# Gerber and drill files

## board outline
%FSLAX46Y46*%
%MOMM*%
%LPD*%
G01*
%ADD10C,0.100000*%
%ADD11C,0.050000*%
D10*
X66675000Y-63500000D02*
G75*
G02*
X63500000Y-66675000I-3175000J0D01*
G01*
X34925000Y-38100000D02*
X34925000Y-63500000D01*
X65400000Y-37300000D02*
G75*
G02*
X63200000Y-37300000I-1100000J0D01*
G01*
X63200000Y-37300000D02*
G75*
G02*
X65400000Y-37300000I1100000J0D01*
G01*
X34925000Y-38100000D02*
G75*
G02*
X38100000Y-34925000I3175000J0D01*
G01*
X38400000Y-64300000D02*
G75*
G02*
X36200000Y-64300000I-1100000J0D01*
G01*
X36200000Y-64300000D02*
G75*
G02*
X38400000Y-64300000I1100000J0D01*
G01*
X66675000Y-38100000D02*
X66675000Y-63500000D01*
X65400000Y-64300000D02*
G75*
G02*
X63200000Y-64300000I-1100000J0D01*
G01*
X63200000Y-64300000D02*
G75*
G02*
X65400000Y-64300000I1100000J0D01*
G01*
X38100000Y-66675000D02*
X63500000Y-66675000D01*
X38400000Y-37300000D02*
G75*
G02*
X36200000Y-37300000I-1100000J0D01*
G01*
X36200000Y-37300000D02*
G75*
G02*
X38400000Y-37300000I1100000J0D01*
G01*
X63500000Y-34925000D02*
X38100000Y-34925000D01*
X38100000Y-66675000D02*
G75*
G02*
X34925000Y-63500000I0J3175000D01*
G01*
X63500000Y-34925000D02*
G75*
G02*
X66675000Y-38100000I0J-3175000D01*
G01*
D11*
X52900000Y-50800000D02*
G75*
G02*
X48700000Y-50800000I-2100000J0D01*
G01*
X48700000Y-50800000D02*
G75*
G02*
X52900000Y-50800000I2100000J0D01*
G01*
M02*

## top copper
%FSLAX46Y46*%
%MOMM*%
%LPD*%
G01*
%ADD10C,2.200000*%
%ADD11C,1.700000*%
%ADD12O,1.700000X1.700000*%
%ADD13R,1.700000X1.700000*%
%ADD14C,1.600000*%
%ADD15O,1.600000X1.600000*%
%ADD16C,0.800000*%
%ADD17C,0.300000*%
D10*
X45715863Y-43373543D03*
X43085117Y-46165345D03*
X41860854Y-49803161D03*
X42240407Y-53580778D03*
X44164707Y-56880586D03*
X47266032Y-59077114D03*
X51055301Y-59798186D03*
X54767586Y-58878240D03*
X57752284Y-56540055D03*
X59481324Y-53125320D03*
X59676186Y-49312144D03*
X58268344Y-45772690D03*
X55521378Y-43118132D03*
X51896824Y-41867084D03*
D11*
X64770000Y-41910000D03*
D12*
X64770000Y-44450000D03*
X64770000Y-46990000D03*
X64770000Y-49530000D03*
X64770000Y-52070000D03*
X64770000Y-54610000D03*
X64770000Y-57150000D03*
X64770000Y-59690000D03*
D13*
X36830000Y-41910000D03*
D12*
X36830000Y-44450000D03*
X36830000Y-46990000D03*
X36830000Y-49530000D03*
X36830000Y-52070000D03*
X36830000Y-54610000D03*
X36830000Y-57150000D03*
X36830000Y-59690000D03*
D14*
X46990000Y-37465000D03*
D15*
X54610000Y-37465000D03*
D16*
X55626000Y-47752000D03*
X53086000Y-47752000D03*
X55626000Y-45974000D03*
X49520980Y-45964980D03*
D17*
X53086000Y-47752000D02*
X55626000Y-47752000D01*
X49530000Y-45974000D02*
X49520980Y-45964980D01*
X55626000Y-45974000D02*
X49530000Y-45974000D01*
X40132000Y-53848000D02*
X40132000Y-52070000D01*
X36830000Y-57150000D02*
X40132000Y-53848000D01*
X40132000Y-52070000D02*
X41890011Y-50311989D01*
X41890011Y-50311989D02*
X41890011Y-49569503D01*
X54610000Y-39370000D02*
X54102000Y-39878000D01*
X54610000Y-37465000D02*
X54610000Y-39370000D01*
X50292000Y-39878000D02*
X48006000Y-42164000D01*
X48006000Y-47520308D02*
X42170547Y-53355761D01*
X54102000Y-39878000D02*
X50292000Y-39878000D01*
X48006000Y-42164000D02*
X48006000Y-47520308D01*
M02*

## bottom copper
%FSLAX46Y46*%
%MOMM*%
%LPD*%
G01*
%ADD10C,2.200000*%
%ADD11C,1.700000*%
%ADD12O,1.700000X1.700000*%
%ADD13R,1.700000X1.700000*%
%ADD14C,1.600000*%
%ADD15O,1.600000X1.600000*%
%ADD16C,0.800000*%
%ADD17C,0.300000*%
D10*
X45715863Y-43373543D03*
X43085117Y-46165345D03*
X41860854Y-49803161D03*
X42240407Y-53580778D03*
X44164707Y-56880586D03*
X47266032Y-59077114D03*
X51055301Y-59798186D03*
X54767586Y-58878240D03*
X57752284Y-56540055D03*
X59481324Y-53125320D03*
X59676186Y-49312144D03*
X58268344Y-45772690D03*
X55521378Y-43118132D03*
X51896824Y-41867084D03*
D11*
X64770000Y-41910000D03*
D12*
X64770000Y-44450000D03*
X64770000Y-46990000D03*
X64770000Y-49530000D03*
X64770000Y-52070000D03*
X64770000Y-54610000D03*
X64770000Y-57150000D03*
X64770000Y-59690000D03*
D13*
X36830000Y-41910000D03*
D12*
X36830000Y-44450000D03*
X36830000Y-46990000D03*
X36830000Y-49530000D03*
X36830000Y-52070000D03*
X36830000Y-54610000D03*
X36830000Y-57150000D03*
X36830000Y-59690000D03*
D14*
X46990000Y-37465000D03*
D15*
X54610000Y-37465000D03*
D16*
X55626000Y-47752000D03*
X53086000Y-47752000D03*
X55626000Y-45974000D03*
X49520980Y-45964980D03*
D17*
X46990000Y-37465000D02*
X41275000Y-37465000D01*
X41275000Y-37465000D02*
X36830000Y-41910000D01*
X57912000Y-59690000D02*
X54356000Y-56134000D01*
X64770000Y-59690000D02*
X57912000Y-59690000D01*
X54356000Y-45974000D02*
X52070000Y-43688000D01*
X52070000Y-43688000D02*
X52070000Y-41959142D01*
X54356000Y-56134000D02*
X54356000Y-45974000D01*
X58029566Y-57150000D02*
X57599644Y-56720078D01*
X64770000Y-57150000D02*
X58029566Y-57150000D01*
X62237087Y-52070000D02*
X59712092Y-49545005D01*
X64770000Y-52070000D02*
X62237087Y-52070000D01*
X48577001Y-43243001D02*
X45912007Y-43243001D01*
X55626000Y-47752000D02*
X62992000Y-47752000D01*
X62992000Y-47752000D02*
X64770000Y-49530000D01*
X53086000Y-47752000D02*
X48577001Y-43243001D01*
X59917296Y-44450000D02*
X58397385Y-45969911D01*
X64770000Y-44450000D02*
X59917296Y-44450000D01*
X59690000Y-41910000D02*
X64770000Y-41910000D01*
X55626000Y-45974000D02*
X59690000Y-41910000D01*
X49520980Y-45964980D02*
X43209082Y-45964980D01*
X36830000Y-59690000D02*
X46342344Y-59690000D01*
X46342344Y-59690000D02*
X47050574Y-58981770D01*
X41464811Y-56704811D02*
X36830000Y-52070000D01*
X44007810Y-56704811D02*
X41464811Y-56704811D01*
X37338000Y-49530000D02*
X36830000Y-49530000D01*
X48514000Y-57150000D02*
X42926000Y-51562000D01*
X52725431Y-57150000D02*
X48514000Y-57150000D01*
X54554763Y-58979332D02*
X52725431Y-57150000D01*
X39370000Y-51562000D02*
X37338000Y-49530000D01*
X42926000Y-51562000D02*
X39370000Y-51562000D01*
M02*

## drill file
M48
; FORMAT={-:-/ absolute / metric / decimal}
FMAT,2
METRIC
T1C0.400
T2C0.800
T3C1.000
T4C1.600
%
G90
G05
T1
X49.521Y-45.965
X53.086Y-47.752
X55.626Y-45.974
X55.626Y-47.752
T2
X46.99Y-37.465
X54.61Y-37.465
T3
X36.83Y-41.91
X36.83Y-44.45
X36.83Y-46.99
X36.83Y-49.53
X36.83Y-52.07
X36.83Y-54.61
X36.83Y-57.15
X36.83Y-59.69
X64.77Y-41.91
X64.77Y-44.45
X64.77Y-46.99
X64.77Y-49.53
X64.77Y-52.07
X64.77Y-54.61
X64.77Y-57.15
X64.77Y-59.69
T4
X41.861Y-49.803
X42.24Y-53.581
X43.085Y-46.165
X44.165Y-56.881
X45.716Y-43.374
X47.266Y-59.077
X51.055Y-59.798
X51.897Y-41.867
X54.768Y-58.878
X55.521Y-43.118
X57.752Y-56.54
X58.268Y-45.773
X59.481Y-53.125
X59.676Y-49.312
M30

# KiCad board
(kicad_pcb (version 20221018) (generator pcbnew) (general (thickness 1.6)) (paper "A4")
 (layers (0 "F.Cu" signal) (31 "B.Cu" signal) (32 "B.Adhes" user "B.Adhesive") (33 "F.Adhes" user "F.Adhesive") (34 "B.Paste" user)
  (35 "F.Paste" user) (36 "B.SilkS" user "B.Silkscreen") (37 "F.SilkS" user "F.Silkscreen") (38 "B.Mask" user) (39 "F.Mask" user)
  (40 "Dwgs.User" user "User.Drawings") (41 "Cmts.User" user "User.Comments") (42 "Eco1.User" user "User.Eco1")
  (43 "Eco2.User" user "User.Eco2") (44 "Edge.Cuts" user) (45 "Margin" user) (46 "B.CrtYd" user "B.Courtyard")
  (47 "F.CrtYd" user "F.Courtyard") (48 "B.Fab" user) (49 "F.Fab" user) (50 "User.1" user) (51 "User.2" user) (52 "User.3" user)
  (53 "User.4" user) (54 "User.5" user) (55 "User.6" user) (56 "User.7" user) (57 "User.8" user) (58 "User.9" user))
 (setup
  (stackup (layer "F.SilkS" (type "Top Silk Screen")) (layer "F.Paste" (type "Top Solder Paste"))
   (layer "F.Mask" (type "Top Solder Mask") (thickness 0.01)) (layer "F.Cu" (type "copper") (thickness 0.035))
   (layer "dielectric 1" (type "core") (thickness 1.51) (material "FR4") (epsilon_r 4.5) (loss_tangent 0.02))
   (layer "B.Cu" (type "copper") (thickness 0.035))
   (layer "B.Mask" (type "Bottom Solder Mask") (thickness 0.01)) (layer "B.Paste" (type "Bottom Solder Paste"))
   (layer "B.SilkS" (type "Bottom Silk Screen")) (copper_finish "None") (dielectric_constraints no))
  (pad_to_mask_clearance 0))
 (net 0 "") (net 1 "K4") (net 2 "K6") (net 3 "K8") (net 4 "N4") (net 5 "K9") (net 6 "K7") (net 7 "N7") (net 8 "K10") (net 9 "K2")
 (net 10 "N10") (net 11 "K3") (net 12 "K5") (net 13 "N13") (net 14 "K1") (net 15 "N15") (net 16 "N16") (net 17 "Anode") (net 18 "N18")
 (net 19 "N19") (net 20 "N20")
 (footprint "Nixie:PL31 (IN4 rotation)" (layer "F.Cu") (at 50.8 50.8 180)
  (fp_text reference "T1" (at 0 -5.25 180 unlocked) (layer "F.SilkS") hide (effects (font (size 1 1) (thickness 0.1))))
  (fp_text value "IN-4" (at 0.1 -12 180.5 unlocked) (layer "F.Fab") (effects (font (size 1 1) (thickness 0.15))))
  (fp_circle (center 0 0) (end 2.09928 -0.054972) (stroke (width 0.05) (type default)) (fill none) (layer "Edge.Cuts"))
  (pad "1" thru_hole circle (at 5.084137 7.426457 353) (size 2.2 2.2) (drill 1.6) (layers "*.Cu" "*.Mask") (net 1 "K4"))
  (pad "2" thru_hole circle (at 7.714883 4.634655 353) (size 2.2 2.2) (drill 1.6) (layers "*.Cu" "*.Mask") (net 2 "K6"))
  (pad "3" thru_hole circle (at 8.939146 0.996839 353) (size 2.2 2.2) (drill 1.6) (layers "*.Cu" "*.Mask") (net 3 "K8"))
  (pad "4" thru_hole circle (at 8.559593 -2.780778 353) (size 2.2 2.2) (drill 1.6) (layers "*.Cu" "*.Mask") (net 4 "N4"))
  (pad "5" thru_hole circle (at 6.635293 -6.080586 353) (size 2.2 2.2) (drill 1.6) (layers "*.Cu" "*.Mask") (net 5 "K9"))
  (pad "6" thru_hole circle (at 3.533968 -8.277114 353) (size 2.2 2.2) (drill 1.6) (layers "*.Cu" "*.Mask") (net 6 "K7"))
  (pad "7" thru_hole circle (at -0.255301 -8.998186 353) (size 2.2 2.2) (drill 1.6) (layers "*.Cu" "*.Mask") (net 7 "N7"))
  (pad "8" thru_hole circle (at -3.967586 -8.07824 353) (size 2.2 2.2) (drill 1.6) (layers "*.Cu" "*.Mask") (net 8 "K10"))
  (pad "9" thru_hole circle (at -6.952284 -5.740055 353) (size 2.2 2.2) (drill 1.6) (layers "*.Cu" "*.Mask") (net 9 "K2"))
  (pad "10" thru_hole circle (at -8.681324 -2.32532 353) (size 2.2 2.2) (drill 1.6) (layers "*.Cu" "*.Mask") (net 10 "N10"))
  (pad "11" thru_hole circle (at -8.876186 1.487856 353) (size 2.2 2.2) (drill 1.6) (layers "*.Cu" "*.Mask") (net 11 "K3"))
  (pad "12" thru_hole circle (at -7.468344 5.02731 353) (size 2.2 2.2) (drill 1.6) (layers "*.Cu" "*.Mask") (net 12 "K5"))
  (pad "13" thru_hole circle (at -4.721378 7.681868 353) (size 2.2 2.2) (drill 1.6) (layers "*.Cu" "*.Mask") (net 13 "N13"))
  (pad "14" thru_hole circle (at -1.096824 8.932916 353) (size 2.2 2.2) (drill 1.6) (layers "*.Cu" "*.Mask") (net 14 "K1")))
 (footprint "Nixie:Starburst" (layer "F.Cu") (at 43 63.25)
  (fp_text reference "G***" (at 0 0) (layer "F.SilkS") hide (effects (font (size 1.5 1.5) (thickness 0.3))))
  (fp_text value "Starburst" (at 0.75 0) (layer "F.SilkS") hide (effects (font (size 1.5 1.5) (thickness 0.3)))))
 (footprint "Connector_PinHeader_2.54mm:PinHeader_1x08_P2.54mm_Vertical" (layer "B.Cu") (at 64.77 41.91 180)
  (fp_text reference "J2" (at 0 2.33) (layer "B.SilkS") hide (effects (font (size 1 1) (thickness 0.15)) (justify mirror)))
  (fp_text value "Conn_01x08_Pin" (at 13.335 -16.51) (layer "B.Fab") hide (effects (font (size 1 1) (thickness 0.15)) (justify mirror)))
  (pad "1" thru_hole circle (at 0 0 180) (size 1.7 1.7) (drill 1) (layers "*.Cu" "*.Mask") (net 2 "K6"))
  (pad "2" thru_hole oval (at 0 -2.54 180) (size 1.7 1.7) (drill 1) (layers "*.Cu" "*.Mask") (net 12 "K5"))
  (pad "3" thru_hole oval (at 0 -5.08 180) (size 1.7 1.7) (drill 1) (layers "*.Cu" "*.Mask") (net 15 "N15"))
  (pad "4" thru_hole oval (at 0 -7.62 180) (size 1.7 1.7) (drill 1) (layers "*.Cu" "*.Mask") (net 1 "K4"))
  (pad "5" thru_hole oval (at 0 -10.16 180) (size 1.7 1.7) (drill 1) (layers "*.Cu" "*.Mask") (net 11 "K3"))
  (pad "6" thru_hole oval (at 0 -12.7 180) (size 1.7 1.7) (drill 1) (layers "*.Cu" "*.Mask") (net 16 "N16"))
  (pad "7" thru_hole oval (at 0 -15.24 180) (size 1.7 1.7) (drill 1) (layers "*.Cu" "*.Mask") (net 9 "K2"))
  (pad "8" thru_hole oval (at 0 -17.78 180) (size 1.7 1.7) (drill 1) (layers "*.Cu" "*.Mask") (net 14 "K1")))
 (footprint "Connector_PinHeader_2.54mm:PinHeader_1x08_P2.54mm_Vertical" (layer "B.Cu") (at 36.83 41.91 180)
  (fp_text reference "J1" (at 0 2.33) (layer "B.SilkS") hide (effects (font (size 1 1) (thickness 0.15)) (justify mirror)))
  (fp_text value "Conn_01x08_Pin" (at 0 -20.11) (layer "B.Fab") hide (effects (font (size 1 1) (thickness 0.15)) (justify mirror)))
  (pad "1" thru_hole rect (at 0 0 180) (size 1.7 1.7) (drill 1) (layers "*.Cu" "*.Mask") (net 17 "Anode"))
  (pad "2" thru_hole oval (at 0 -2.54 180) (size 1.7 1.7) (drill 1) (layers "*.Cu" "*.Mask") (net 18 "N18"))
  (pad "3" thru_hole oval (at 0 -5.08 180) (size 1.7 1.7) (drill 1) (layers "*.Cu" "*.Mask") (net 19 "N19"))
  (pad "4" thru_hole oval (at 0 -7.62 180) (size 1.7 1.7) (drill 1) (layers "*.Cu" "*.Mask") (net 8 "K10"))
  (pad "5" thru_hole oval (at 0 -10.16 180) (size 1.7 1.7) (drill 1) (layers "*.Cu" "*.Mask") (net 5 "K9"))
  (pad "6" thru_hole oval (at 0 -12.7 180) (size 1.7 1.7) (drill 1) (layers "*.Cu" "*.Mask") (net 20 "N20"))
  (pad "7" thru_hole oval (at 0 -15.24 180) (size 1.7 1.7) (drill 1) (layers "*.Cu" "*.Mask") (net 3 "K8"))
  (pad "8" thru_hole oval (at 0 -17.78 180) (size 1.7 1.7) (drill 1) (layers "*.Cu" "*.Mask") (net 6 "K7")))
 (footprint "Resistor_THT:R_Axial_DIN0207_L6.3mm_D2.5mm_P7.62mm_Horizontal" (layer "B.Cu") (at 46.99 37.465)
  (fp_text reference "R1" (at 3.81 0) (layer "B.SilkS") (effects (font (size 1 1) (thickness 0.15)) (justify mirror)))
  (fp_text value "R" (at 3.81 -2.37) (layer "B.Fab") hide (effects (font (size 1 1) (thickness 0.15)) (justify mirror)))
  (pad "1" thru_hole circle (at 0 0) (size 1.6 1.6) (drill 0.8) (layers "*.Cu" "*.Mask") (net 17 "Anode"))
  (pad "2" thru_hole oval (at 7.62 0) (size 1.6 1.6) (drill 0.8) (layers "*.Cu" "*.Mask") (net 4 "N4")))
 (gr_arc (start 66.675 63.5) (mid 65.745064 65.745064) (end 63.5 66.675) (stroke (width 0.1) (type default)) (layer "Edge.Cuts"))
 (gr_line (start 34.925 38.1) (end 34.925 63.5) (stroke (width 0.1) (type default)) (layer "Edge.Cuts"))
 (gr_circle (center 64.3 37.3) (end 65.4 37.3) (stroke (width 0.1) (type default)) (fill none) (layer "Edge.Cuts"))
 (gr_arc (start 34.925 38.1) (mid 35.854936 35.854936) (end 38.1 34.925) (stroke (width 0.1) (type default)) (layer "Edge.Cuts"))
 (gr_circle (center 37.3 64.3) (end 38.4 64.3) (stroke (width 0.1) (type default)) (fill none) (layer "Edge.Cuts"))
 (gr_line (start 66.675 38.1) (end 66.675 63.5) (stroke (width 0.1) (type default)) (layer "Edge.Cuts"))
 (gr_circle (center 64.3 64.3) (end 65.4 64.3) (stroke (width 0.1) (type default)) (fill none) (layer "Edge.Cuts"))
 (gr_line (start 38.1 66.675) (end 63.5 66.675) (stroke (width 0.1) (type default)) (layer "Edge.Cuts"))
 (gr_circle (center 37.3 37.3) (end 38.4 37.3) (stroke (width 0.1) (type default)) (fill none) (layer "Edge.Cuts"))
 (gr_line (start 63.5 34.925) (end 38.1 34.925) (stroke (width 0.1) (type default)) (layer "Edge.Cuts"))
 (gr_arc (start 38.1 66.675) (mid 35.854936 65.745064) (end 34.925 63.5) (stroke (width 0.1) (type default)) (layer "Edge.Cuts"))
 (gr_arc (start 63.5 34.925) (mid 65.745064 35.854936) (end 66.675 38.1) (stroke (width 0.1) (type default)) (layer "Edge.Cuts"))
 (segment (start 46.99 37.465) (end 41.275 37.465) (width 0.3) (layer "B.Cu") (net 17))
 (segment (start 41.275 37.465) (end 36.83 41.91) (width 0.3) (layer "B.Cu") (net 17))
 (segment (start 57.912 59.69) (end 54.356 56.134) (width 0.3) (layer "B.Cu") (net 14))
 (segment (start 64.77 59.69) (end 57.912 59.69) (width 0.3) (layer "B.Cu") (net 14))
 (segment (start 54.356 45.974) (end 52.07 43.688) (width 0.3) (layer "B.Cu") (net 14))
 (segment (start 52.07 43.688) (end 52.07 41.959142) (width 0.3) (layer "B.Cu") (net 14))
 (segment (start 54.356 56.134) (end 54.356 45.974) (width 0.3) (layer "B.Cu") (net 14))
 (segment (start 58.029566 57.15) (end 57.599644 56.720078) (width 0.3) (layer "B.Cu") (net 9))
 (segment (start 64.77 57.15) (end 58.029566 57.15) (width 0.3) (layer "B.Cu") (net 9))
 (segment (start 62.237087 52.07) (end 59.712092 49.545005) (width 0.3) (layer "B.Cu") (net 11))
 (segment (start 64.77 52.07) (end 62.237087 52.07) (width 0.3) (layer "B.Cu") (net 11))
 (segment (start 53.086 47.752) (end 55.626 47.752) (width 0.3) (layer "F.Cu") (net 1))
 (via (at 55.626 47.752) (size 0.8) (drill 0.4) (layers "F.Cu" "B.Cu") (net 1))
 (via (at 53.086 47.752) (size 0.8) (drill 0.4) (layers "F.Cu" "B.Cu") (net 1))
 (segment (start 48.577001 43.243001) (end 45.912007 43.243001) (width 0.3) (layer "B.Cu") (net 1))
 (segment (start 55.626 47.752) (end 62.992 47.752) (width 0.3) (layer "B.Cu") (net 1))
 (segment (start 62.992 47.752) (end 64.77 49.53) (width 0.3) (layer "B.Cu") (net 1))
 (segment (start 53.086 47.752) (end 48.577001 43.243001) (width 0.3) (layer "B.Cu") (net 1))
 (segment (start 59.917296 44.45) (end 58.397385 45.969911) (width 0.3) (layer "B.Cu") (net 12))
 (segment (start 64.77 44.45) (end 59.917296 44.45) (width 0.3) (layer "B.Cu") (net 12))
 (segment (start 49.53 45.974) (end 49.52098 45.96498) (width 0.3) (layer "F.Cu") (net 2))
 (segment (start 55.626 45.974) (end 49.53 45.974) (width 0.3) (layer "F.Cu") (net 2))
 (via (at 55.626 45.974) (size 0.8) (drill 0.4) (layers "F.Cu" "B.Cu") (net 2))
 (via (at 49.52098 45.96498) (size 0.8) (drill 0.4) (layers "F.Cu" "B.Cu") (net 2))
 (segment (start 59.69 41.91) (end 64.77 41.91) (width 0.3) (layer "B.Cu") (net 2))
 (segment (start 55.626 45.974) (end 59.69 41.91) (width 0.3) (layer "B.Cu") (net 2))
 (segment (start 49.52098 45.96498) (end 43.209082 45.96498) (width 0.3) (layer "B.Cu") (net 2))
 (segment (start 36.83 59.69) (end 46.342344 59.69) (width 0.3) (layer "B.Cu") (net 6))
 (segment (start 46.342344 59.69) (end 47.050574 58.98177) (width 0.3) (layer "B.Cu") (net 6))
 (segment (start 40.132 53.848) (end 40.132 52.07) (width 0.3) (layer "F.Cu") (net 3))
 (segment (start 36.83 57.15) (end 40.132 53.848) (width 0.3) (layer "F.Cu") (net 3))
 (segment (start 40.132 52.07) (end 41.890011 50.311989) (width 0.3) (layer "F.Cu") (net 3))
 (segment (start 41.890011 50.311989) (end 41.890011 49.569503) (width 0.3) (layer "F.Cu") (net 3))
 (segment (start 41.464811 56.704811) (end 36.83 52.07) (width 0.3) (layer "B.Cu") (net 5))
 (segment (start 44.00781 56.704811) (end 41.464811 56.704811) (width 0.3) (layer "B.Cu") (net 5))
 (segment (start 37.338 49.53) (end 36.83 49.53) (width 0.3) (layer "B.Cu") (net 8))
 (segment (start 48.514 57.15) (end 42.926 51.562) (width 0.3) (layer "B.Cu") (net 8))
 (segment (start 52.725431 57.15) (end 48.514 57.15) (width 0.3) (layer "B.Cu") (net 8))
 (segment (start 54.554763 58.979332) (end 52.725431 57.15) (width 0.3) (layer "B.Cu") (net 8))
 (segment (start 39.37 51.562) (end 37.338 49.53) (width 0.3) (layer "B.Cu") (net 8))
 (segment (start 42.926 51.562) (end 39.37 51.562) (width 0.3) (layer "B.Cu") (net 8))
 (segment (start 54.61 39.37) (end 54.102 39.878) (width 0.3) (layer "F.Cu") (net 4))
 (segment (start 54.61 37.465) (end 54.61 39.37) (width 0.3) (layer "F.Cu") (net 4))
 (segment (start 50.292 39.878) (end 48.006 42.164) (width 0.3) (layer "F.Cu") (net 4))
 (segment (start 48.006 47.520308) (end 42.170547 53.355761) (width 0.3) (layer "F.Cu") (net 4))
 (segment (start 54.102 39.878) (end 50.292 39.878) (width 0.3) (layer "F.Cu") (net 4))
 (segment (start 48.006 42.164) (end 48.006 47.520308) (width 0.3) (layer "F.Cu") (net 4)))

